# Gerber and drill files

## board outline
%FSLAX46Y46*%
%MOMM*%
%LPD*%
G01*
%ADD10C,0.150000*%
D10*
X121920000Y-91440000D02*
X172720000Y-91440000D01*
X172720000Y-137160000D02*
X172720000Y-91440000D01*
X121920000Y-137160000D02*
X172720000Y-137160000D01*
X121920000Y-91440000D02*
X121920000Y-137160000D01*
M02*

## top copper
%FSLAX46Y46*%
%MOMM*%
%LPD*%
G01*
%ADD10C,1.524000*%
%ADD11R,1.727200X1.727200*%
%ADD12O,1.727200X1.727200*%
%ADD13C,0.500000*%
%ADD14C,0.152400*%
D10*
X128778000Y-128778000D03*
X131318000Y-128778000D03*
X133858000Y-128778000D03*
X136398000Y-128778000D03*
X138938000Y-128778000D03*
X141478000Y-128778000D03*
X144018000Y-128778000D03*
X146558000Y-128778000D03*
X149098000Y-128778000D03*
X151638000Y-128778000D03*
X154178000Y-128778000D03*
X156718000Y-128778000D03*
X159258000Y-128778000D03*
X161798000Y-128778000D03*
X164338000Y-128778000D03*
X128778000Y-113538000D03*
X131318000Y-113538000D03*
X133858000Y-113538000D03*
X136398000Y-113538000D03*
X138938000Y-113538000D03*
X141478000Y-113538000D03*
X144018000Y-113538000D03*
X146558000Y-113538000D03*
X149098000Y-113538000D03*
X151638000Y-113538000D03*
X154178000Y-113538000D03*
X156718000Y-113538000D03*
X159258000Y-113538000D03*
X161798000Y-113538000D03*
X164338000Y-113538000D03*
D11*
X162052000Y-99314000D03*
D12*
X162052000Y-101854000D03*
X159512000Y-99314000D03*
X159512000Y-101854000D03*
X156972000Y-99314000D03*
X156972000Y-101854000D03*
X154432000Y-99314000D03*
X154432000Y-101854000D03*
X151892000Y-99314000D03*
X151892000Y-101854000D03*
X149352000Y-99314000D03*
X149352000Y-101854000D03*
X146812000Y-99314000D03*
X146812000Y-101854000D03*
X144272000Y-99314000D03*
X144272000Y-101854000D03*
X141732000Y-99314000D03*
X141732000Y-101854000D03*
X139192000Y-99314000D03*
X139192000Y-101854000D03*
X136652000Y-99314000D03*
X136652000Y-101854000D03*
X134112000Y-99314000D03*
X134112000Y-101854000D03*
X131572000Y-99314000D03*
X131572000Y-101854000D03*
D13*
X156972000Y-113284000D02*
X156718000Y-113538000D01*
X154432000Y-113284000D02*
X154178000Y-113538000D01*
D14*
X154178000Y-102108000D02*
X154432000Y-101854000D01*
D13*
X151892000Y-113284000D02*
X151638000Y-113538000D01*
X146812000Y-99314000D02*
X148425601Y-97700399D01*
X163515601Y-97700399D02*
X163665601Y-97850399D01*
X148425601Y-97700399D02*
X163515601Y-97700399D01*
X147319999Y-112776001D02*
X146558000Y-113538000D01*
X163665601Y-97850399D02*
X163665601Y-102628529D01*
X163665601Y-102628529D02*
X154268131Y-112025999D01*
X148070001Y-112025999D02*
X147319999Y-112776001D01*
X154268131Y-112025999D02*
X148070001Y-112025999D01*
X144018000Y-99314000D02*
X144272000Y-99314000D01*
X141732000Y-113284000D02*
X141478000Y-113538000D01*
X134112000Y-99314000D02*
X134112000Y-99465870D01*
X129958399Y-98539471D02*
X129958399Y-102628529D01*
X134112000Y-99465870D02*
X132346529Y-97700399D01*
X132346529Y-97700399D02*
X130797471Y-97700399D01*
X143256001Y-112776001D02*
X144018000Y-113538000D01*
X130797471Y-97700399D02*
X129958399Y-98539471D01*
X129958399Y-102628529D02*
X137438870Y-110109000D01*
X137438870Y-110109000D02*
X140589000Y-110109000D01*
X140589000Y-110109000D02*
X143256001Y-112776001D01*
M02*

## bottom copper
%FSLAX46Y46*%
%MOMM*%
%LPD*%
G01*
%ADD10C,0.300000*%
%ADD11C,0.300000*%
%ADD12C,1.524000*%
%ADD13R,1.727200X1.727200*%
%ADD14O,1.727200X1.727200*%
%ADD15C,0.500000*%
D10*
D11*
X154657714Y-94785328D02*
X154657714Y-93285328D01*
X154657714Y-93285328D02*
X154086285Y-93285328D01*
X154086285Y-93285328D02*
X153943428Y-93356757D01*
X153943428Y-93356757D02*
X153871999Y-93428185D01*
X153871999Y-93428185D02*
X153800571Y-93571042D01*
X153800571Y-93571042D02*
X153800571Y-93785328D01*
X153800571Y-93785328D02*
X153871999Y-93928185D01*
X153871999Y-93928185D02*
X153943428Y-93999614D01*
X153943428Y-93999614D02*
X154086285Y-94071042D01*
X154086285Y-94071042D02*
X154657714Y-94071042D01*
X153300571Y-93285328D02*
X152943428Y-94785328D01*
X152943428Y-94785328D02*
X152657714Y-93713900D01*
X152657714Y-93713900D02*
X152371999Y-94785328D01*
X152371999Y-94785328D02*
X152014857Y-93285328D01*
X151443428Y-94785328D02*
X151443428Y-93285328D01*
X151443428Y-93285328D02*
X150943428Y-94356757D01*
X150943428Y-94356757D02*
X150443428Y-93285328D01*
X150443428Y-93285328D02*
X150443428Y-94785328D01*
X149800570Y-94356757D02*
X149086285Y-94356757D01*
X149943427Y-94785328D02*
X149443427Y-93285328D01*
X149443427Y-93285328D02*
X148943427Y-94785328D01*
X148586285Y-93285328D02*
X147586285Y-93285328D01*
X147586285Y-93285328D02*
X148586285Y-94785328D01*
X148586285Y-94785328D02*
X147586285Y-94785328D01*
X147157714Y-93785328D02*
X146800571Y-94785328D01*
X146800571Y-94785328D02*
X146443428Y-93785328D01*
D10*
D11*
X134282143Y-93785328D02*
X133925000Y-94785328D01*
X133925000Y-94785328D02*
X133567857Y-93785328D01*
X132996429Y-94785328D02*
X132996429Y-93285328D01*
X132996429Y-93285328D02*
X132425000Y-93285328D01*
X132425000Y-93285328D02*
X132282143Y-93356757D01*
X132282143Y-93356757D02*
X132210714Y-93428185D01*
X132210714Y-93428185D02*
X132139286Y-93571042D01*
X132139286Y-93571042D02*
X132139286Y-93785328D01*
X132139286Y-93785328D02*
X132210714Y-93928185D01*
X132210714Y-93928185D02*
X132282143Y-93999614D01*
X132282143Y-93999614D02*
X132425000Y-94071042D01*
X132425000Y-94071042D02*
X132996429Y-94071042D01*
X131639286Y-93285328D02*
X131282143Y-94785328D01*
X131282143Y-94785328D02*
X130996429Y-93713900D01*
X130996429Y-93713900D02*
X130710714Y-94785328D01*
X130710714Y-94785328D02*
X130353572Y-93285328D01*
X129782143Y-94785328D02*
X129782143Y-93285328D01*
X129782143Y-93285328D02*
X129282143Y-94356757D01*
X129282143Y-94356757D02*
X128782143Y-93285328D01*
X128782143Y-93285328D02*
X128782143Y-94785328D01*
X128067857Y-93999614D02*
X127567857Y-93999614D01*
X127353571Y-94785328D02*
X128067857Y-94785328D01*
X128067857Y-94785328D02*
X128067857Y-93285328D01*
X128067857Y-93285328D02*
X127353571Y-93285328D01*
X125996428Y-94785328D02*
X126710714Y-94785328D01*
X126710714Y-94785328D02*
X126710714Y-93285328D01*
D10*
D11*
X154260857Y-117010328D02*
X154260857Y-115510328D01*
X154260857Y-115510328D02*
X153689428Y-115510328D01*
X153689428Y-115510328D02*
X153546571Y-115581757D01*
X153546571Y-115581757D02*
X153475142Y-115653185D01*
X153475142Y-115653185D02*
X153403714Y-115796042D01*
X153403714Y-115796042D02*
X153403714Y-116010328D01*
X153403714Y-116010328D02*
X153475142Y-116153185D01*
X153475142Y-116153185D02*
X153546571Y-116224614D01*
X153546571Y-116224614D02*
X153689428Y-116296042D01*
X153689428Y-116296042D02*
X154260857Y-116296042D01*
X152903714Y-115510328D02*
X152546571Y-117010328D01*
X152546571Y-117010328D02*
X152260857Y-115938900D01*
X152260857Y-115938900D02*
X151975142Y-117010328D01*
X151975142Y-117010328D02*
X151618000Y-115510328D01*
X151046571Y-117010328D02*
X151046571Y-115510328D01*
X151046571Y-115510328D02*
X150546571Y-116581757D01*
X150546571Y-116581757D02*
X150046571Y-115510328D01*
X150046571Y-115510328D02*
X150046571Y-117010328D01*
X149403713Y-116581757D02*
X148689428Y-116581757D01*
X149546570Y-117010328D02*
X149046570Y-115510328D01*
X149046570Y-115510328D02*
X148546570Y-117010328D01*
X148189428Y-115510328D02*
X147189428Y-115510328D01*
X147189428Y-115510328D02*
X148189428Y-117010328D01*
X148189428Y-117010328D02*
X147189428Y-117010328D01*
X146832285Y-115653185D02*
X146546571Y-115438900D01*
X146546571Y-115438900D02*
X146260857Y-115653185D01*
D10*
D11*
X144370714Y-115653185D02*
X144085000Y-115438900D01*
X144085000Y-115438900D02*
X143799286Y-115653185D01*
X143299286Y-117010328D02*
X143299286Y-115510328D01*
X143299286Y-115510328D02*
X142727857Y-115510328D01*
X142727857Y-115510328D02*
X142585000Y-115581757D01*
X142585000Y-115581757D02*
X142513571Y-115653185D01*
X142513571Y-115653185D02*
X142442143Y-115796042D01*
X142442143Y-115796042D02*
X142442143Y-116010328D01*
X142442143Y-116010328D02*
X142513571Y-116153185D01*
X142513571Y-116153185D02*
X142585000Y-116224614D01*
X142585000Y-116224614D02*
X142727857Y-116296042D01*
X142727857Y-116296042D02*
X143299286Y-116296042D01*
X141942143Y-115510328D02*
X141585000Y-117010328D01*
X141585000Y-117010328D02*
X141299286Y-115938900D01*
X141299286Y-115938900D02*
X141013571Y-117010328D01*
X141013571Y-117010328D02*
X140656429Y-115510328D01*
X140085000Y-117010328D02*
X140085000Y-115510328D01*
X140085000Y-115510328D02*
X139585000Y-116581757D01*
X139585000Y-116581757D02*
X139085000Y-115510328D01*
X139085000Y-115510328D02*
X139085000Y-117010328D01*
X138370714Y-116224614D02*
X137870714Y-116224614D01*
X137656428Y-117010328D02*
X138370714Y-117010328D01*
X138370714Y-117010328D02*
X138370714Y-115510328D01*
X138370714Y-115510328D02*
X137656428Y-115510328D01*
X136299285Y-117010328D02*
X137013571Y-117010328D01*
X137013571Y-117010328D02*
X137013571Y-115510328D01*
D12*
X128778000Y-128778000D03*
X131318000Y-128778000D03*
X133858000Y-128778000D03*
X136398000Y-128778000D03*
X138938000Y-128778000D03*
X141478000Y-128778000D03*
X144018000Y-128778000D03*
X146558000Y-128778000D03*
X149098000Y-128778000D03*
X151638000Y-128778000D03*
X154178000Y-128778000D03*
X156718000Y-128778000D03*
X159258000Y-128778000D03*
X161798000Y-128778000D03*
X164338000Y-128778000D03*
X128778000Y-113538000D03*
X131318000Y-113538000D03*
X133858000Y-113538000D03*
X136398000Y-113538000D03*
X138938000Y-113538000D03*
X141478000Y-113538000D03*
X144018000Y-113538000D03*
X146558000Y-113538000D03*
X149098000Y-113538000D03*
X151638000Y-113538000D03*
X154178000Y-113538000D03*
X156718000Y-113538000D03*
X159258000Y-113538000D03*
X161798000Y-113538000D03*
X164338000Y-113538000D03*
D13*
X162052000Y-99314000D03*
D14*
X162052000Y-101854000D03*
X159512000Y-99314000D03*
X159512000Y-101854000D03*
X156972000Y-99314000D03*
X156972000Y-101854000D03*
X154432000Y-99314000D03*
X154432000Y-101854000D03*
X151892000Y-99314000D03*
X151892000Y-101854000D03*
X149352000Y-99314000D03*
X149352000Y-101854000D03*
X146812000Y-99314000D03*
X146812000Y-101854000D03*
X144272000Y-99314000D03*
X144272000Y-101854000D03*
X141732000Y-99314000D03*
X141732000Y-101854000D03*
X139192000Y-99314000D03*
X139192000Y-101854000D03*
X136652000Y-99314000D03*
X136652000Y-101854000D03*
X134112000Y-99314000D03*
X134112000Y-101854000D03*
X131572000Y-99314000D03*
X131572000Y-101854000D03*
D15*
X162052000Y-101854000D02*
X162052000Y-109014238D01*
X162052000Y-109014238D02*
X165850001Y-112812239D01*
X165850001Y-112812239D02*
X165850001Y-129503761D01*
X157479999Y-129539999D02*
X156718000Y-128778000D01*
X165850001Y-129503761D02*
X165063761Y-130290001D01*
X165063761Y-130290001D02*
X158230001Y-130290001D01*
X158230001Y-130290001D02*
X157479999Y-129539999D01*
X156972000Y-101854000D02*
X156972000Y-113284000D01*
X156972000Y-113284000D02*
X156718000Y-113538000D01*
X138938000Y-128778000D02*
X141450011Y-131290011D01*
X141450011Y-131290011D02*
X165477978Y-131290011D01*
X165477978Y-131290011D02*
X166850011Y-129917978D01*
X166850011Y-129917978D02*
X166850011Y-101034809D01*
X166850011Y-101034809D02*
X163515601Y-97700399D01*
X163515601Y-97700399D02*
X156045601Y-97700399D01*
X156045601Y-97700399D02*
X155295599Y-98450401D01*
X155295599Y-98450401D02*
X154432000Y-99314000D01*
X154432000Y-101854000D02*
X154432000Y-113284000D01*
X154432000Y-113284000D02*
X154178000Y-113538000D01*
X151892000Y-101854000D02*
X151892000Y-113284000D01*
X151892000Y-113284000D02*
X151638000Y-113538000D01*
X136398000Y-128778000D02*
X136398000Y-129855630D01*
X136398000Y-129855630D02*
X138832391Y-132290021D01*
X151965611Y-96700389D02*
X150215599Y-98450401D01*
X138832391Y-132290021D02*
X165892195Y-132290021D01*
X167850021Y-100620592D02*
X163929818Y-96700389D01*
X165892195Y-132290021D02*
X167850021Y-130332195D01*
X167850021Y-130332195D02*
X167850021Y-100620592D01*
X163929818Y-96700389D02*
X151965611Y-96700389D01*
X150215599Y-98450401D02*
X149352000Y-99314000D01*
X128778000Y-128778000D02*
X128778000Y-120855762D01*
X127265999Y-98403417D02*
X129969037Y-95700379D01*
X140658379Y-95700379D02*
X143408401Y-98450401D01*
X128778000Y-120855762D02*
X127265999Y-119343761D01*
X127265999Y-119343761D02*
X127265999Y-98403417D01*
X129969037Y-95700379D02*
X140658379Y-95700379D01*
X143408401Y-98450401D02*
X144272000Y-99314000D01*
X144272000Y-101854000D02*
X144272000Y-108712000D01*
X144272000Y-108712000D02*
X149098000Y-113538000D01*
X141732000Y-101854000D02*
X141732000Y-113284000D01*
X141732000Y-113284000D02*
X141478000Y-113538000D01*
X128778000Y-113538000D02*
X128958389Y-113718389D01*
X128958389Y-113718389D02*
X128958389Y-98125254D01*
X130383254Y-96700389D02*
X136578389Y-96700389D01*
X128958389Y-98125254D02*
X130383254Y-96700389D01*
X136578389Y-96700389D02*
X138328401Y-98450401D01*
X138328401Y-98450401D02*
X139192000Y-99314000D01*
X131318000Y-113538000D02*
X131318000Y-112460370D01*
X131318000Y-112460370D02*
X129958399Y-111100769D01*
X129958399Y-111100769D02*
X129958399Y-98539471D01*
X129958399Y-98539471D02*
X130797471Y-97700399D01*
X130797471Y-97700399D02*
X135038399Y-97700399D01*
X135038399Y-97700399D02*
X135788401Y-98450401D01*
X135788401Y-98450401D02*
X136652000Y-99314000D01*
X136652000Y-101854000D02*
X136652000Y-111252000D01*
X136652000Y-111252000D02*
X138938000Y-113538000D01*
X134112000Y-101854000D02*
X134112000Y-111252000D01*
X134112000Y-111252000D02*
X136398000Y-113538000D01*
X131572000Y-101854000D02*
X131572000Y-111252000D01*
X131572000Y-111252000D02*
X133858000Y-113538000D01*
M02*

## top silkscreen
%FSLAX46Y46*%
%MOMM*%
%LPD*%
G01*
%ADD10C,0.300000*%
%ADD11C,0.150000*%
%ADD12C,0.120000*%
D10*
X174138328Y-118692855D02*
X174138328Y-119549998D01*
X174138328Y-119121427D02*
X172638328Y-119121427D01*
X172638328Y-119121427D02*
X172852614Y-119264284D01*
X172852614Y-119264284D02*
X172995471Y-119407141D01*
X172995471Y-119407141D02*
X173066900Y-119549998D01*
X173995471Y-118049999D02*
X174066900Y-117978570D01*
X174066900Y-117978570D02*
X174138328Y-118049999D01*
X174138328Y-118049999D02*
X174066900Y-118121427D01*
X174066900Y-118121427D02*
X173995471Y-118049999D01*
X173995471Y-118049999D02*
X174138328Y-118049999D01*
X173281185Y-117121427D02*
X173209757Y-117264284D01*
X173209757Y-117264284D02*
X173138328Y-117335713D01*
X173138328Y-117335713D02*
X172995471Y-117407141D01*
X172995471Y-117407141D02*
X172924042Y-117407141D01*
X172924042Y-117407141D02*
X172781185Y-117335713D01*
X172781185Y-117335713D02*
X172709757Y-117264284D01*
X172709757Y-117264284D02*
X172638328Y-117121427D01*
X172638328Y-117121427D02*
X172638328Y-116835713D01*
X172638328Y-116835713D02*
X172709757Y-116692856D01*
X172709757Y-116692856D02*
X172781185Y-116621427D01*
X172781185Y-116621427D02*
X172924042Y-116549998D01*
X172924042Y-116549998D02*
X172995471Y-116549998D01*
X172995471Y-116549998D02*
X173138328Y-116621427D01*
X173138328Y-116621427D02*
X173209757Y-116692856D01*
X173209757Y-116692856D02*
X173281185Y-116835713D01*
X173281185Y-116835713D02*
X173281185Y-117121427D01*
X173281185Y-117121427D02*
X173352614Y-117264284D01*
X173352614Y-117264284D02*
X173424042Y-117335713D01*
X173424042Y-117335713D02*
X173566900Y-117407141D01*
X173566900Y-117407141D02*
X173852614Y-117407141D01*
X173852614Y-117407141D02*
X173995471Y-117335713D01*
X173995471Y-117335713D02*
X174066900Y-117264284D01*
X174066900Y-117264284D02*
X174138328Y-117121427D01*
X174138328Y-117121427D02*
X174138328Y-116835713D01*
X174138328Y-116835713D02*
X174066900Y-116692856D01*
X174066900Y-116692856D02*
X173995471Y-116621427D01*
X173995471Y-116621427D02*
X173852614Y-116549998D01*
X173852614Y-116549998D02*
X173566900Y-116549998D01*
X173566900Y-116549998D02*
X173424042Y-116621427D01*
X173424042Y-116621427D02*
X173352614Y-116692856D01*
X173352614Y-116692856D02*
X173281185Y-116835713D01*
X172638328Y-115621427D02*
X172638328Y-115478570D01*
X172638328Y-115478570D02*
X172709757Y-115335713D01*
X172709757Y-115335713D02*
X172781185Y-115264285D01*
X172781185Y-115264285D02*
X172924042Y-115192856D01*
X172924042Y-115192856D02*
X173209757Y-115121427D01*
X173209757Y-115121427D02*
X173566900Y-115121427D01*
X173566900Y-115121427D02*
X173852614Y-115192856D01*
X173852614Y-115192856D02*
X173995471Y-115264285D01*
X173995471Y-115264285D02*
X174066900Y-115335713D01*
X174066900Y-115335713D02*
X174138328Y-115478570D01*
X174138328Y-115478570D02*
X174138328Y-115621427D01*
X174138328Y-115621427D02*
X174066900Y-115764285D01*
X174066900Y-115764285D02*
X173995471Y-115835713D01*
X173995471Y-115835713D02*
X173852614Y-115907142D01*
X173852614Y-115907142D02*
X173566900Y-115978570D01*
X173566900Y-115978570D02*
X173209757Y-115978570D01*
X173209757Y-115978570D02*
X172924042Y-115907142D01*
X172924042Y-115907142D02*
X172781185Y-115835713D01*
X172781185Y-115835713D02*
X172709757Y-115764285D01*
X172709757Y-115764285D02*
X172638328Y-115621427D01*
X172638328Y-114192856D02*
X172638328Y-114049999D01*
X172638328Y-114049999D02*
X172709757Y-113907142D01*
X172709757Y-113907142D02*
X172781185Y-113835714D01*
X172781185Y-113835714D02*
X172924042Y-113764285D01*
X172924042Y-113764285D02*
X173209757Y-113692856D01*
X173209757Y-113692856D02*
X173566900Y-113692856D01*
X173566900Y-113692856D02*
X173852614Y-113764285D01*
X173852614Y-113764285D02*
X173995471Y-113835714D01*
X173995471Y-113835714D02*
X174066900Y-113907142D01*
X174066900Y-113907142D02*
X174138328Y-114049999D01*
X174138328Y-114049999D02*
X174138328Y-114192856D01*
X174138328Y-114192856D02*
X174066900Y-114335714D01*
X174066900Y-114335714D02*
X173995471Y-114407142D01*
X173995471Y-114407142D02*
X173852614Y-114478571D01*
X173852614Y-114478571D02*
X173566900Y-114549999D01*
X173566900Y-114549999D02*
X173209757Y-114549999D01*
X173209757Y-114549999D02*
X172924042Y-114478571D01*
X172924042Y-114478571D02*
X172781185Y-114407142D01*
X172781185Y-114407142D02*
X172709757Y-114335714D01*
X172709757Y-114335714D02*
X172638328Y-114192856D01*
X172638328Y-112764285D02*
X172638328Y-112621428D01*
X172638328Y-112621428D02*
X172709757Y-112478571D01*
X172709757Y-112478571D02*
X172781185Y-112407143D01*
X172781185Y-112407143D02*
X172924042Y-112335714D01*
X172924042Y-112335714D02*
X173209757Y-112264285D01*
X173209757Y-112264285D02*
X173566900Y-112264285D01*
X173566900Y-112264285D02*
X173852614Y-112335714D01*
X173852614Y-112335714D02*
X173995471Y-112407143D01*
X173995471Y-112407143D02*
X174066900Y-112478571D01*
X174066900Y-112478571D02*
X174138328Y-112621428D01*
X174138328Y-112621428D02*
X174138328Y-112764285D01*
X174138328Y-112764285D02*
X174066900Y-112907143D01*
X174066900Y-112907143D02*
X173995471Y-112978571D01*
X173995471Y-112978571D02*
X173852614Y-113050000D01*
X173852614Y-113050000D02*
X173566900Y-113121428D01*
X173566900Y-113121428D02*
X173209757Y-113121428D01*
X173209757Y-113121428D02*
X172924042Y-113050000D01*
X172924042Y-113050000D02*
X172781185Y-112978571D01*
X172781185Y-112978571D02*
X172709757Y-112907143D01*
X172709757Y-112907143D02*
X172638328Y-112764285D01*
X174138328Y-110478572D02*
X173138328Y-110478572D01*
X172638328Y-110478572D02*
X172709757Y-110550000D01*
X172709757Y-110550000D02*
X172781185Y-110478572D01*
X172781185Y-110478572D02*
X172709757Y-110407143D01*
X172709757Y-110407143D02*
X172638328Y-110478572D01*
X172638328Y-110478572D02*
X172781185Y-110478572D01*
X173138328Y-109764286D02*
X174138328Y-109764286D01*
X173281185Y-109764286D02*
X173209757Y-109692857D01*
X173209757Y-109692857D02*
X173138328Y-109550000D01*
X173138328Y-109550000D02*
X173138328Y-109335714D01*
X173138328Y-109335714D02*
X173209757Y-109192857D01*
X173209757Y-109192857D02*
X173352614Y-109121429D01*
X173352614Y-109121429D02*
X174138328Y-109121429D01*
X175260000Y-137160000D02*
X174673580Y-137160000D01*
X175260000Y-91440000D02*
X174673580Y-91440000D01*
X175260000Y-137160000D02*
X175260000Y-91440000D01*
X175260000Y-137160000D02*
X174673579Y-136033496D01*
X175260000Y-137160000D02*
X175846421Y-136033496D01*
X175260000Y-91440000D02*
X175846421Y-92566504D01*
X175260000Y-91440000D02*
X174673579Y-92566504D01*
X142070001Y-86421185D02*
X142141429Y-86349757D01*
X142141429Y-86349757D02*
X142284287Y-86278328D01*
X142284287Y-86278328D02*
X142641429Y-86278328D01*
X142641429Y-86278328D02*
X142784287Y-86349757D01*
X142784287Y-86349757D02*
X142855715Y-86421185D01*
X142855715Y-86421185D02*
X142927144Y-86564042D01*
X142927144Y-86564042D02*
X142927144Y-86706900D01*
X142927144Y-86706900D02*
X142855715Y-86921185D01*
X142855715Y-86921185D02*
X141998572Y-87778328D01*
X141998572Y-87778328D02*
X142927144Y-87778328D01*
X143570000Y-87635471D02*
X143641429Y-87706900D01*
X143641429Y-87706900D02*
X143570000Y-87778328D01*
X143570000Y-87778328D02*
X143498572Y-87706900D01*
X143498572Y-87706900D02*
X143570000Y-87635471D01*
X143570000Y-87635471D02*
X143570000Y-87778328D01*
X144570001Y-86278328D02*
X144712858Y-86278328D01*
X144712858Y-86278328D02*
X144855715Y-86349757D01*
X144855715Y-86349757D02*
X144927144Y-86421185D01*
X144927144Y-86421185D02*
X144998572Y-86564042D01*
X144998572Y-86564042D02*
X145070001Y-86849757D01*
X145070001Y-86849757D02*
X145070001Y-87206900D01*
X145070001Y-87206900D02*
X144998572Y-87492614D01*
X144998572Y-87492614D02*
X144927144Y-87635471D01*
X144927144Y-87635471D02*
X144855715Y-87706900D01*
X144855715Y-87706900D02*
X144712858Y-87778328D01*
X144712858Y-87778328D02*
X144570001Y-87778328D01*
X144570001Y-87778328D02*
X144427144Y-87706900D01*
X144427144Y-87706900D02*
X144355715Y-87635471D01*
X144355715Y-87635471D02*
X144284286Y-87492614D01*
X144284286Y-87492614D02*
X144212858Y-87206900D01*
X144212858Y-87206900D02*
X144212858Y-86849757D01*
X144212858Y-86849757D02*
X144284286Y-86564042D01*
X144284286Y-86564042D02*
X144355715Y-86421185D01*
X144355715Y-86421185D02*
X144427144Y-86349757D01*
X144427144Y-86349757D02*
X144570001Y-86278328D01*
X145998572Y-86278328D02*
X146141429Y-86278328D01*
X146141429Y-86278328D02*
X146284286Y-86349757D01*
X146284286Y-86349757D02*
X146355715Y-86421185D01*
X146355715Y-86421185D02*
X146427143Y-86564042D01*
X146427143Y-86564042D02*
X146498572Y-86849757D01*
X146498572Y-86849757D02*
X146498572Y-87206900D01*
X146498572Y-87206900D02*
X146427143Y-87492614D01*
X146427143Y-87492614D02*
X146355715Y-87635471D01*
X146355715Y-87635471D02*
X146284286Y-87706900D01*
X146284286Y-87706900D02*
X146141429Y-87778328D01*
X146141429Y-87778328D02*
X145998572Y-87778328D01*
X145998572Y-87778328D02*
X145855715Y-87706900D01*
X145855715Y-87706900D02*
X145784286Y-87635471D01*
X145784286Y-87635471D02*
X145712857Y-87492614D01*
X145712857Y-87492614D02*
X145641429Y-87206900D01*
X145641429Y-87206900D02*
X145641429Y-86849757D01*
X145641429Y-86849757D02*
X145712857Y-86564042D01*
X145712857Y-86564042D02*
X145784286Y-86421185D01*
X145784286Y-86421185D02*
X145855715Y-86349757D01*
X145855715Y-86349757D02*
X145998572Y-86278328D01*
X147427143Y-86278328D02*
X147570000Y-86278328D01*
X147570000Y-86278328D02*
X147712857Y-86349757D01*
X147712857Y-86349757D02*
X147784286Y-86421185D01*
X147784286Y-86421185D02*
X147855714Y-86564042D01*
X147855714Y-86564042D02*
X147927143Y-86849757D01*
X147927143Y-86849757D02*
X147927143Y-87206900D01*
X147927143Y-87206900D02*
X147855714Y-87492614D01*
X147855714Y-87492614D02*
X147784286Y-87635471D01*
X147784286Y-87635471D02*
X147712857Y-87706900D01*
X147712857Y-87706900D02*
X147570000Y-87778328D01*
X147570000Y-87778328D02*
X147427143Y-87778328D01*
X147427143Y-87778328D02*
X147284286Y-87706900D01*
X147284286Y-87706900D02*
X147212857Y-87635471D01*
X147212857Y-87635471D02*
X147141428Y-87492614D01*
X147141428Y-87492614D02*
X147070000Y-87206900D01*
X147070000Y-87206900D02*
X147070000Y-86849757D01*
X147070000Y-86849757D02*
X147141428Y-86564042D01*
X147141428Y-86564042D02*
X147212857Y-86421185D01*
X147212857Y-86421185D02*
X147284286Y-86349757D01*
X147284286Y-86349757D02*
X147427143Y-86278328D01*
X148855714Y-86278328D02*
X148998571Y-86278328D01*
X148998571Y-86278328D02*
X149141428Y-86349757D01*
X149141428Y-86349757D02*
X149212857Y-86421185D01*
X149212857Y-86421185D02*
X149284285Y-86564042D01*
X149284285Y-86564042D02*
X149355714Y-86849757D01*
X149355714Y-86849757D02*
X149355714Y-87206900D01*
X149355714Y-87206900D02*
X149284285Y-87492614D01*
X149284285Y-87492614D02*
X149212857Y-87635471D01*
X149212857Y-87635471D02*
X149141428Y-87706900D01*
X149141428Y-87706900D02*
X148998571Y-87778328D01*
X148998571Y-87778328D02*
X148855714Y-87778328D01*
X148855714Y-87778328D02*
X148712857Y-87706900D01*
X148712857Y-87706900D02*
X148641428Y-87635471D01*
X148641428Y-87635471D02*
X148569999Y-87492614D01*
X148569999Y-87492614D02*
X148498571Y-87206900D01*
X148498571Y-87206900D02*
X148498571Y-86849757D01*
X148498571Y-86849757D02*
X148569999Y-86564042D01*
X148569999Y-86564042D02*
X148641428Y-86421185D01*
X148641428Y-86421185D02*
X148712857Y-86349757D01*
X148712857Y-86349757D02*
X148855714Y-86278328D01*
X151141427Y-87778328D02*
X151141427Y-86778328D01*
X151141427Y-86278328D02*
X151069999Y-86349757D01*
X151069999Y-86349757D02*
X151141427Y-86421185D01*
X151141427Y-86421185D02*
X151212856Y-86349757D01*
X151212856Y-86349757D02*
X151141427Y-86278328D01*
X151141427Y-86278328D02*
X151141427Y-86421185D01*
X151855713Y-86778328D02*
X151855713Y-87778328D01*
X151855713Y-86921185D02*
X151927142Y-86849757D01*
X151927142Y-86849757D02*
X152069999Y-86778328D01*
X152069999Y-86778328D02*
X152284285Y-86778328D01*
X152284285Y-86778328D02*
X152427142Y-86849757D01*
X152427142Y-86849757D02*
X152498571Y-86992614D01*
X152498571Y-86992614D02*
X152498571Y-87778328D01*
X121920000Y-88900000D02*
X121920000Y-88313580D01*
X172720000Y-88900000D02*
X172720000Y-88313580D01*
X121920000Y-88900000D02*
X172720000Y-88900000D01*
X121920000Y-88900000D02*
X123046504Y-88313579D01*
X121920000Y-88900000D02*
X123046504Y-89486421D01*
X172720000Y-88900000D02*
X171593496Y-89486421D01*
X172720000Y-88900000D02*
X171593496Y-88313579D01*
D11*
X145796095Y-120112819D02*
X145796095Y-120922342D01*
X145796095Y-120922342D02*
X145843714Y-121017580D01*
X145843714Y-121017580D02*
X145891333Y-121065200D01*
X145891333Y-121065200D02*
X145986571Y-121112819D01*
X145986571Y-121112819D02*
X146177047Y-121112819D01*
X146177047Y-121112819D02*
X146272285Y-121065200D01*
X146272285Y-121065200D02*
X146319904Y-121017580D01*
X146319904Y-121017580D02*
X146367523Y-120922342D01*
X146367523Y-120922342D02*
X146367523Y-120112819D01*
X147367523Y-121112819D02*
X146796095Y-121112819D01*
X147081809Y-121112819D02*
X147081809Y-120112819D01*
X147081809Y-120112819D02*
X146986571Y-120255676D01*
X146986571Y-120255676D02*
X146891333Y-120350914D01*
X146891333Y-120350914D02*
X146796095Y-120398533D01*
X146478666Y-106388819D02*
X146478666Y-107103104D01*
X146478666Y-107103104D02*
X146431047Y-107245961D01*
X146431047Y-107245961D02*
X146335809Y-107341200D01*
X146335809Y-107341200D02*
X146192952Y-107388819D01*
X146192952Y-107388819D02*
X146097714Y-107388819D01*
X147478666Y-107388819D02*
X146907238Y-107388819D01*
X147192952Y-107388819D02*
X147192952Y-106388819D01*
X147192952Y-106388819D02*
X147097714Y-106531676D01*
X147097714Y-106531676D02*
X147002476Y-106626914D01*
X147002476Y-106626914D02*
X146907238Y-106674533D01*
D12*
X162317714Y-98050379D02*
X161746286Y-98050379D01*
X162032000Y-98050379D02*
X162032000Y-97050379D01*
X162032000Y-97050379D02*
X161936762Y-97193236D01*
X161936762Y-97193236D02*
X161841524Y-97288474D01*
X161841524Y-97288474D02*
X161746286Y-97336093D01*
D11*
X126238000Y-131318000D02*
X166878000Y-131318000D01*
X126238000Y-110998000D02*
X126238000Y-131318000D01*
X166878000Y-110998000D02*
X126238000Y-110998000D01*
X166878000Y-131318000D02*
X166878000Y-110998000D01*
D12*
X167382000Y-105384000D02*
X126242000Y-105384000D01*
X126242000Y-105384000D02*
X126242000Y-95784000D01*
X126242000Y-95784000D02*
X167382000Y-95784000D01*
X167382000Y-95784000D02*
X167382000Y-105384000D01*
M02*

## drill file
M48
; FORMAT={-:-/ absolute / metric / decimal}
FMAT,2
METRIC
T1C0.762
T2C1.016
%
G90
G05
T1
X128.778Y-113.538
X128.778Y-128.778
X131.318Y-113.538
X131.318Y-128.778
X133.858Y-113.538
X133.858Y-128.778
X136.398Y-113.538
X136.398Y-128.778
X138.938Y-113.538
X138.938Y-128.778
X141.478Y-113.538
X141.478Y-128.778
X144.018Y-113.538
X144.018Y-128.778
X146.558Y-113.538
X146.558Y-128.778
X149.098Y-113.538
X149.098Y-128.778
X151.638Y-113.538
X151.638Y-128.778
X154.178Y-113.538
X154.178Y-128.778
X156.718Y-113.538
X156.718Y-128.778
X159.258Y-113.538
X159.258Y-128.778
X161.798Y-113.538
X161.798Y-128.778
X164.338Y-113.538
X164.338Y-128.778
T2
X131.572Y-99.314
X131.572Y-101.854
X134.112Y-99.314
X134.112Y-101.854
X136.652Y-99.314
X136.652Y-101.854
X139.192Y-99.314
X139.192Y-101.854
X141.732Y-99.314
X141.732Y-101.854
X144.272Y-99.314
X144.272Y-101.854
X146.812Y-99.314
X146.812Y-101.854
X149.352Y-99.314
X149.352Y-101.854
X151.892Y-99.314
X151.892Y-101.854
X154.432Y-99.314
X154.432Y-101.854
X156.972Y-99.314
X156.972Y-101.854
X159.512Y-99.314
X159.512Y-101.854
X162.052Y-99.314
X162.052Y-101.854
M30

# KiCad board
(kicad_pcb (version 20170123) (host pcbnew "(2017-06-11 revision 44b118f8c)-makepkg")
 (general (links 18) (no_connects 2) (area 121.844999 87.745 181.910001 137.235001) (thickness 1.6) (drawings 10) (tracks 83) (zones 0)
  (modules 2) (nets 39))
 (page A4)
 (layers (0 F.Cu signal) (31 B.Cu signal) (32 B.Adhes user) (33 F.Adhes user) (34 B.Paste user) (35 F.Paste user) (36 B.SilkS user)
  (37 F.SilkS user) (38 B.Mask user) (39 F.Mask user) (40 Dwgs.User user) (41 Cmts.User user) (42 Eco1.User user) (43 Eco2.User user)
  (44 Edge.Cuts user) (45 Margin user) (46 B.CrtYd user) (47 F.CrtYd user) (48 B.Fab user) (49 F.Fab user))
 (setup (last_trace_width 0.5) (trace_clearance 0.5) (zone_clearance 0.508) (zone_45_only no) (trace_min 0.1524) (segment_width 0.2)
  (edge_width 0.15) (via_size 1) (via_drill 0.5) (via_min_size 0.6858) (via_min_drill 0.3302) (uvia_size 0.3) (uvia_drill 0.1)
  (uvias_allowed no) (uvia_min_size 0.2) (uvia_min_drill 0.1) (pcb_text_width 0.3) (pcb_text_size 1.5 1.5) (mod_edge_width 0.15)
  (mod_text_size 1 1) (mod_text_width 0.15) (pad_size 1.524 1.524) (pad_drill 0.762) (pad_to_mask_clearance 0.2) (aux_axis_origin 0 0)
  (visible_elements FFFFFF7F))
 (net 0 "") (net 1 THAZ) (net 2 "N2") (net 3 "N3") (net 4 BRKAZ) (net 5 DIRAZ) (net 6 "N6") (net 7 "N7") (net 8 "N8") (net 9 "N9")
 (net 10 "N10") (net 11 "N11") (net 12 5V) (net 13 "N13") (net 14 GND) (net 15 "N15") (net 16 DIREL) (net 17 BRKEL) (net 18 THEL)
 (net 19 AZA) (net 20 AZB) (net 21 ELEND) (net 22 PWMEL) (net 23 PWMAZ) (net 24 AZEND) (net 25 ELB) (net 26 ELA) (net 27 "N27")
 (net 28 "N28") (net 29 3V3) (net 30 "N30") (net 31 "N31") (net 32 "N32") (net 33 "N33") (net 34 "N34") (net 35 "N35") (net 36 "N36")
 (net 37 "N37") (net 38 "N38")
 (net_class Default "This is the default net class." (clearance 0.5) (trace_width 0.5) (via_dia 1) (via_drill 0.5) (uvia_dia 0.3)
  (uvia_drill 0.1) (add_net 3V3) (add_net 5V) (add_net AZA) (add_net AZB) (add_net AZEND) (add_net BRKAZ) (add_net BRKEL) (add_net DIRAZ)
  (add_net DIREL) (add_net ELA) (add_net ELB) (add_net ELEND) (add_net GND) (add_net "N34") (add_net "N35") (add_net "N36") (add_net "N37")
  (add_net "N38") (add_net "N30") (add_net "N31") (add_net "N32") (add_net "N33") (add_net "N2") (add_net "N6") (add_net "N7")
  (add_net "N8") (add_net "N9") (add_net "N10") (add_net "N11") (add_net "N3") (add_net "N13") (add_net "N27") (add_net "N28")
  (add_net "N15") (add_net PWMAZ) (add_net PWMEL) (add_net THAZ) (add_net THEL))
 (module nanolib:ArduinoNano (layer F.Cu) (at 146.558 121.158 180)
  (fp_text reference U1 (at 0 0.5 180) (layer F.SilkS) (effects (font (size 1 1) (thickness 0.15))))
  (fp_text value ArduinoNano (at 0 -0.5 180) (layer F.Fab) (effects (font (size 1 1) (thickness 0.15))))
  (fp_line (start 20.32 -10.16) (end -20.32 -10.16) (layer F.SilkS) (width 0.15))
  (fp_line (start 20.32 10.16) (end 20.32 -10.16) (layer F.SilkS) (width 0.15))
  (fp_line (start -20.32 10.16) (end 20.32 10.16) (layer F.SilkS) (width 0.15))
  (fp_line (start -20.32 -10.16) (end -20.32 10.16) (layer F.SilkS) (width 0.15))
  (pad D13 thru_hole circle (at 17.78 -7.62 180) (size 1.524 1.524) (drill 0.762) (layers *.Cu *.Mask) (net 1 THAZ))
  (pad 3V3 thru_hole circle (at 15.24 -7.62 180) (size 1.524 1.524) (drill 0.762) (layers *.Cu *.Mask) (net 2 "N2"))
  (pad REF thru_hole circle (at 12.7 -7.62 180) (size 1.524 1.524) (drill 0.762) (layers *.Cu *.Mask) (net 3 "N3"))
  (pad A0 thru_hole circle (at 10.16 -7.62 180) (size 1.524 1.524) (drill 0.762) (layers *.Cu *.Mask) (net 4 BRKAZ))
  (pad A1 thru_hole circle (at 7.62 -7.62 180) (size 1.524 1.524) (drill 0.762) (layers *.Cu *.Mask) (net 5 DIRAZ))
  (pad A2 thru_hole circle (at 5.08 -7.62 180) (size 1.524 1.524) (drill 0.762) (layers *.Cu *.Mask) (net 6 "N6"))
  (pad A3 thru_hole circle (at 2.54 -7.62 180) (size 1.524 1.524) (drill 0.762) (layers *.Cu *.Mask) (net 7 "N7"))
  (pad A4 thru_hole circle (at 0 -7.62 180) (size 1.524 1.524) (drill 0.762) (layers *.Cu *.Mask) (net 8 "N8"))
  (pad A5 thru_hole circle (at -2.54 -7.62 180) (size 1.524 1.524) (drill 0.762) (layers *.Cu *.Mask) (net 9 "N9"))
  (pad A6 thru_hole circle (at -5.08 -7.62 180) (size 1.524 1.524) (drill 0.762) (layers *.Cu *.Mask) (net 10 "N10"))
  (pad A7 thru_hole circle (at -7.62 -7.62 180) (size 1.524 1.524) (drill 0.762) (layers *.Cu *.Mask) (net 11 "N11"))
  (pad 5V thru_hole circle (at -10.16 -7.62 180) (size 1.524 1.524) (drill 0.762) (layers *.Cu *.Mask) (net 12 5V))
  (pad RST thru_hole circle (at -12.7 -7.62 180) (size 1.524 1.524) (drill 0.762) (layers *.Cu *.Mask) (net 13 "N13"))
  (pad GND thru_hole circle (at -15.24 -7.62 180) (size 1.524 1.524) (drill 0.762) (layers *.Cu *.Mask) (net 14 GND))
  (pad VIN thru_hole circle (at -17.78 -7.62 180) (size 1.524 1.524) (drill 0.762) (layers *.Cu *.Mask) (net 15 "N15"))
  (pad D12 thru_hole circle (at 17.78 7.62 180) (size 1.524 1.524) (drill 0.762) (layers *.Cu *.Mask) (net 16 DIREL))
  (pad D11 thru_hole circle (at 15.24 7.62 180) (size 1.524 1.524) (drill 0.762) (layers *.Cu *.Mask) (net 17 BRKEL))
  (pad D10 thru_hole circle (at 12.7 7.62 180) (size 1.524 1.524) (drill 0.762) (layers *.Cu *.Mask) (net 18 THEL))
  (pad D9 thru_hole circle (at 10.16 7.62 180) (size 1.524 1.524) (drill 0.762) (layers *.Cu *.Mask) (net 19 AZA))
  (pad D8 thru_hole circle (at 7.62 7.62 180) (size 1.524 1.524) (drill 0.762) (layers *.Cu *.Mask) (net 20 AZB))
  (pad D7 thru_hole circle (at 5.08 7.62 180) (size 1.524 1.524) (drill 0.762) (layers *.Cu *.Mask) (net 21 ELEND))
  (pad D6 thru_hole circle (at 2.54 7.62 180) (size 1.524 1.524) (drill 0.762) (layers *.Cu *.Mask) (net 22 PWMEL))
  (pad D5 thru_hole circle (at 0 7.62 180) (size 1.524 1.524) (drill 0.762) (layers *.Cu *.Mask) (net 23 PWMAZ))
  (pad D4 thru_hole circle (at -2.54 7.62 180) (size 1.524 1.524) (drill 0.762) (layers *.Cu *.Mask) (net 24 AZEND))
  (pad D3 thru_hole circle (at -5.08 7.62 180) (size 1.524 1.524) (drill 0.762) (layers *.Cu *.Mask) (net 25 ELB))
  (pad D2 thru_hole circle (at -7.62 7.62 180) (size 1.524 1.524) (drill 0.762) (layers *.Cu *.Mask) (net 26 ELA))
  (pad GND thru_hole circle (at -10.16 7.62 180) (size 1.524 1.524) (drill 0.762) (layers *.Cu *.Mask) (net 14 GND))
  (pad RST thru_hole circle (at -12.7 7.62 180) (size 1.524 1.524) (drill 0.762) (layers *.Cu *.Mask) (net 13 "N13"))
  (pad RX0 thru_hole circle (at -15.24 7.62 180) (size 1.524 1.524) (drill 0.762) (layers *.Cu *.Mask) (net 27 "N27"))
  (pad TX1 thru_hole circle (at -17.78 7.62 180) (size 1.524 1.524) (drill 0.762) (layers *.Cu *.Mask) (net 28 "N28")))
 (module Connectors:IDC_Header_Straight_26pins (layer F.Cu) (at 162.052 99.314 180)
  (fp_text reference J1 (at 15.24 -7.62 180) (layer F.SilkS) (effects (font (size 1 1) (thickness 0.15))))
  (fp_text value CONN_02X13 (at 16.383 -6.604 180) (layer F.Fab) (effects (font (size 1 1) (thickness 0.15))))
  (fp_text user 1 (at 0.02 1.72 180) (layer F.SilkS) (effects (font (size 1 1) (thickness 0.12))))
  (fp_line (start -5.33 -6.07) (end 35.81 -6.07) (layer F.SilkS) (width 0.12))
  (fp_line (start 35.81 -6.07) (end 35.81 3.53) (layer F.SilkS) (width 0.12))
  (fp_line (start 35.81 3.53) (end -5.33 3.53) (layer F.SilkS) (width 0.12))
  (fp_line (start -5.33 3.53) (end -5.33 -6.07) (layer F.SilkS) (width 0.12))
  (pad 1 thru_hole rect (at 0 0 180) (size 1.7272 1.7272) (drill 1.016) (layers *.Cu *.Mask) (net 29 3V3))
  (pad 2 thru_hole oval (at 0 -2.54 180) (size 1.7272 1.7272) (drill 1.016) (layers *.Cu *.Mask) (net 12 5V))
  (pad 3 thru_hole oval (at 2.54 0 180) (size 1.7272 1.7272) (drill 1.016) (layers *.Cu *.Mask) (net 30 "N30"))
  (pad 4 thru_hole oval (at 2.54 -2.54 180) (size 1.7272 1.7272) (drill 1.016) (layers *.Cu *.Mask) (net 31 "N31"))
  (pad 5 thru_hole oval (at 5.08 0 180) (size 1.7272 1.7272) (drill 1.016) (layers *.Cu *.Mask) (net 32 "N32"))
  (pad 6 thru_hole oval (at 5.08 -2.54 180) (size 1.7272 1.7272) (drill 1.016) (layers *.Cu *.Mask) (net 14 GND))
  (pad 7 thru_hole oval (at 7.62 0 180) (size 1.7272 1.7272) (drill 1.016) (layers *.Cu *.Mask) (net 5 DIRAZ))
  (pad 8 thru_hole oval (at 7.62 -2.54 180) (size 1.7272 1.7272) (drill 1.016) (layers *.Cu *.Mask) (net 26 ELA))
  (pad 9 thru_hole oval (at 10.16 0 180) (size 1.7272 1.7272) (drill 1.016) (layers *.Cu *.Mask) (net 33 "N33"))
  (pad 10 thru_hole oval (at 10.16 -2.54 180) (size 1.7272 1.7272) (drill 1.016) (layers *.Cu *.Mask) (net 25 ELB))
  (pad 11 thru_hole oval (at 12.7 0 180) (size 1.7272 1.7272) (drill 1.016) (layers *.Cu *.Mask) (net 4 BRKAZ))
  (pad 12 thru_hole oval (at 12.7 -2.54 180) (size 1.7272 1.7272) (drill 1.016) (layers *.Cu *.Mask) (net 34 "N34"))
  (pad 13 thru_hole oval (at 15.24 0 180) (size 1.7272 1.7272) (drill 1.016) (layers *.Cu *.Mask) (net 23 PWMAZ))
  (pad 14 thru_hole oval (at 15.24 -2.54 180) (size 1.7272 1.7272) (drill 1.016) (layers *.Cu *.Mask) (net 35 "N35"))
  (pad 15 thru_hole oval (at 17.78 0 180) (size 1.7272 1.7272) (drill 1.016) (layers *.Cu *.Mask) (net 1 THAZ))
  (pad 16 thru_hole oval (at 17.78 -2.54 180) (size 1.7272 1.7272) (drill 1.016) (layers *.Cu *.Mask) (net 24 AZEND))
  (pad 17 thru_hole oval (at 20.32 0 180) (size 1.7272 1.7272) (drill 1.016) (layers *.Cu *.Mask) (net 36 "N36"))
  (pad 18 thru_hole oval (at 20.32 -2.54 180) (size 1.7272 1.7272) (drill 1.016) (layers *.Cu *.Mask) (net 21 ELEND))
  (pad 19 thru_hole oval (at 22.86 0 180) (size 1.7272 1.7272) (drill 1.016) (layers *.Cu *.Mask) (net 16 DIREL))
  (pad 20 thru_hole oval (at 22.86 -2.54 180) (size 1.7272 1.7272) (drill 1.016) (layers *.Cu *.Mask) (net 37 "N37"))
  (pad 21 thru_hole oval (at 25.4 0 180) (size 1.7272 1.7272) (drill 1.016) (layers *.Cu *.Mask) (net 17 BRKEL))
  (pad 22 thru_hole oval (at 25.4 -2.54 180) (size 1.7272 1.7272) (drill 1.016) (layers *.Cu *.Mask) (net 20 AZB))
  (pad 23 thru_hole oval (at 27.94 0 180) (size 1.7272 1.7272) (drill 1.016) (layers *.Cu *.Mask) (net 22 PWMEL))
  (pad 24 thru_hole oval (at 27.94 -2.54 180) (size 1.7272 1.7272) (drill 1.016) (layers *.Cu *.Mask) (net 19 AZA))
  (pad 25 thru_hole oval (at 30.48 0 180) (size 1.7272 1.7272) (drill 1.016) (layers *.Cu *.Mask) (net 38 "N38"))
  (pad 26 thru_hole oval (at 30.48 -2.54 180) (size 1.7272 1.7272) (drill 1.016) (layers *.Cu *.Mask) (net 18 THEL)))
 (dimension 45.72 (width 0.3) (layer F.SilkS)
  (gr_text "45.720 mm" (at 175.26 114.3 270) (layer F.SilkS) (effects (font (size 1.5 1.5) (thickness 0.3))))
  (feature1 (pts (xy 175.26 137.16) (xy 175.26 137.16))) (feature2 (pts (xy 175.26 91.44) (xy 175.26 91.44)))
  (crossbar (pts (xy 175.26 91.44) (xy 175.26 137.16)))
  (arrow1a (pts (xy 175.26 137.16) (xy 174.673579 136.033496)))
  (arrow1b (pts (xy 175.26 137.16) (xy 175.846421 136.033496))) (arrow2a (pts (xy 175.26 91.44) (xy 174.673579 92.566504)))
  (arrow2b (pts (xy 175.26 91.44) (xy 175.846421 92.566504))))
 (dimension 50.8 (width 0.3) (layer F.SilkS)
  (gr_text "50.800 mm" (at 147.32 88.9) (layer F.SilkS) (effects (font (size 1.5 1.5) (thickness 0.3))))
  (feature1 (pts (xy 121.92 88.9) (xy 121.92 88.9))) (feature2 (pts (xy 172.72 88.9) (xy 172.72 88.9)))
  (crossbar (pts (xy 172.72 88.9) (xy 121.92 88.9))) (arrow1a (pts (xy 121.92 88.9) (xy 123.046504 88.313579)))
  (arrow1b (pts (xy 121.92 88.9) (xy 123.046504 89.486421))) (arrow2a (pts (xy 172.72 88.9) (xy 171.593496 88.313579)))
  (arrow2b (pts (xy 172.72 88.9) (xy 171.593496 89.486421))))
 (gr_line (start 121.92 91.44) (end 172.72 91.44) (layer Edge.Cuts) (width 0.15))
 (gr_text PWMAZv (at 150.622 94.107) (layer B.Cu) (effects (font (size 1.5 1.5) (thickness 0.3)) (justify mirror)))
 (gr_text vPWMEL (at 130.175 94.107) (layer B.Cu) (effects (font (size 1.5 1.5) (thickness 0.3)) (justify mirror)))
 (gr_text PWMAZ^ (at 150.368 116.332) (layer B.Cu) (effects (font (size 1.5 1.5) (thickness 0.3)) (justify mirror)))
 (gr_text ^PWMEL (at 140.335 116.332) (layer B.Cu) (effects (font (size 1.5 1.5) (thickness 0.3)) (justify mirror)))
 (gr_line (start 172.72 137.16) (end 172.72 91.44) (layer Edge.Cuts) (width 0.15))
 (gr_line (start 121.92 137.16) (end 172.72 137.16) (layer Edge.Cuts) (width 0.15))
 (gr_line (start 121.92 91.44) (end 121.92 137.16) (layer Edge.Cuts) (width 0.15))
 (segment (start 162.052 101.854) (end 162.052 109.014238) (width 0.5) (layer B.Cu) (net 12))
 (segment (start 162.052 109.014238) (end 165.850001 112.812239) (width 0.5) (layer B.Cu) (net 12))
 (segment (start 165.850001 112.812239) (end 165.850001 129.503761) (width 0.5) (layer B.Cu) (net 12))
 (segment (start 157.479999 129.539999) (end 156.718 128.778) (width 0.5) (layer B.Cu) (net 12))
 (segment (start 165.850001 129.503761) (end 165.063761 130.290001) (width 0.5) (layer B.Cu) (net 12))
 (segment (start 165.063761 130.290001) (end 158.230001 130.290001) (width 0.5) (layer B.Cu) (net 12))
 (segment (start 158.230001 130.290001) (end 157.479999 129.539999) (width 0.5) (layer B.Cu) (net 12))
 (segment (start 156.972 101.854) (end 156.972 113.284) (width 0.5) (layer B.Cu) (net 14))
 (segment (start 156.972 113.284) (end 156.718 113.538) (width 0.5) (layer B.Cu) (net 14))
 (segment (start 156.972 113.284) (end 156.718 113.538) (width 0.5) (layer F.Cu) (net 14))
 (segment (start 138.938 128.778) (end 141.450011 131.290011) (width 0.5) (layer B.Cu) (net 5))
 (segment (start 141.450011 131.290011) (end 165.477978 131.290011) (width 0.5) (layer B.Cu) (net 5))
 (segment (start 165.477978 131.290011) (end 166.850011 129.917978) (width 0.5) (layer B.Cu) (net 5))
 (segment (start 166.850011 129.917978) (end 166.850011 101.034809) (width 0.5) (layer B.Cu) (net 5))
 (segment (start 166.850011 101.034809) (end 163.515601 97.700399) (width 0.5) (layer B.Cu) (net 5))
 (segment (start 163.515601 97.700399) (end 156.045601 97.700399) (width 0.5) (layer B.Cu) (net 5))
 (segment (start 156.045601 97.700399) (end 155.295599 98.450401) (width 0.5) (layer B.Cu) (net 5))
 (segment (start 155.295599 98.450401) (end 154.432 99.314) (width 0.5) (layer B.Cu) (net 5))
 (segment (start 154.432 101.854) (end 154.432 113.284) (width 0.5) (layer B.Cu) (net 26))
 (segment (start 154.432 113.284) (end 154.178 113.538) (width 0.5) (layer B.Cu) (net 26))
 (segment (start 154.432 113.284) (end 154.178 113.538) (width 0.5) (layer F.Cu) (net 26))
 (segment (start 154.178 102.108) (end 154.432 101.854) (width 0.1524) (layer F.Cu) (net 26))
 (segment (start 151.892 101.854) (end 151.892 113.284) (width 0.5) (layer B.Cu) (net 25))
 (segment (start 151.892 113.284) (end 151.638 113.538) (width 0.5) (layer B.Cu) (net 25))
 (segment (start 151.892 113.284) (end 151.638 113.538) (width 0.5) (layer F.Cu) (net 25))
 (segment (start 136.398 128.778) (end 136.398 129.85563) (width 0.5) (layer B.Cu) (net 4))
 (segment (start 136.398 129.85563) (end 138.832391 132.290021) (width 0.5) (layer B.Cu) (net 4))
 (segment (start 151.965611 96.700389) (end 150.215599 98.450401) (width 0.5) (layer B.Cu) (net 4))
 (segment (start 138.832391 132.290021) (end 165.892195 132.290021) (width 0.5) (layer B.Cu) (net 4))
 (segment (start 167.850021 100.620592) (end 163.929818 96.700389) (width 0.5) (layer B.Cu) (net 4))
 (segment (start 165.892195 132.290021) (end 167.850021 130.332195) (width 0.5) (layer B.Cu) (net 4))
 (segment (start 167.850021 130.332195) (end 167.850021 100.620592) (width 0.5) (layer B.Cu) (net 4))
 (segment (start 163.929818 96.700389) (end 151.965611 96.700389) (width 0.5) (layer B.Cu) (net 4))
 (segment (start 150.215599 98.450401) (end 149.352 99.314) (width 0.5) (layer B.Cu) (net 4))
 (segment (start 146.812 99.314) (end 148.425601 97.700399) (width 0.5) (layer F.Cu) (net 23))
 (segment (start 163.515601 97.700399) (end 163.665601 97.850399) (width 0.5) (layer F.Cu) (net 23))
 (segment (start 148.425601 97.700399) (end 163.515601 97.700399) (width 0.5) (layer F.Cu) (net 23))
 (segment (start 147.319999 112.776001) (end 146.558 113.538) (width 0.5) (layer F.Cu) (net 23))
 (segment (start 163.665601 97.850399) (end 163.665601 102.628529) (width 0.5) (layer F.Cu) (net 23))
 (segment (start 163.665601 102.628529) (end 154.268131 112.025999) (width 0.5) (layer F.Cu) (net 23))
 (segment (start 148.070001 112.025999) (end 147.319999 112.776001) (width 0.5) (layer F.Cu) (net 23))
 (segment (start 154.268131 112.025999) (end 148.070001 112.025999) (width 0.5) (layer F.Cu) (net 23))
 (segment (start 128.778 128.778) (end 128.778 120.855762) (width 0.5) (layer B.Cu) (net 1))
 (segment (start 127.265999 98.403417) (end 129.969037 95.700379) (width 0.5) (layer B.Cu) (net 1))
 (segment (start 140.658379 95.700379) (end 143.408401 98.450401) (width 0.5) (layer B.Cu) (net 1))
 (segment (start 128.778 120.855762) (end 127.265999 119.343761) (width 0.5) (layer B.Cu) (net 1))
 (segment (start 127.265999 119.343761) (end 127.265999 98.403417) (width 0.5) (layer B.Cu) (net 1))
 (segment (start 129.969037 95.700379) (end 140.658379 95.700379) (width 0.5) (layer B.Cu) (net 1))
 (segment (start 143.408401 98.450401) (end 144.272 99.314) (width 0.5) (layer B.Cu) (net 1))
 (segment (start 144.018 99.314) (end 144.272 99.314) (width 0.5) (layer F.Cu) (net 1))
 (segment (start 144.272 101.854) (end 144.272 108.712) (width 0.5) (layer B.Cu) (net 24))
 (segment (start 144.272 108.712) (end 149.098 113.538) (width 0.5) (layer B.Cu) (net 24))
 (segment (start 141.732 101.854) (end 141.732 113.284) (width 0.5) (layer B.Cu) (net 21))
 (segment (start 141.732 113.284) (end 141.478 113.538) (width 0.5) (layer B.Cu) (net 21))
 (segment (start 141.732 113.284) (end 141.478 113.538) (width 0.5) (layer F.Cu) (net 21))
 (segment (start 128.778 113.538) (end 128.958389 113.718389) (width 0.5) (layer B.Cu) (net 16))
 (segment (start 128.958389 113.718389) (end 128.958389 98.125254) (width 0.5) (layer B.Cu) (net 16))
 (segment (start 130.383254 96.700389) (end 136.578389 96.700389) (width 0.5) (layer B.Cu) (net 16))
 (segment (start 128.958389 98.125254) (end 130.383254 96.700389) (width 0.5) (layer B.Cu) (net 16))
 (segment (start 136.578389 96.700389) (end 138.328401 98.450401) (width 0.5) (layer B.Cu) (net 16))
 (segment (start 138.328401 98.450401) (end 139.192 99.314) (width 0.5) (layer B.Cu) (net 16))
 (segment (start 131.318 113.538) (end 131.318 112.46037) (width 0.5) (layer B.Cu) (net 17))
 (segment (start 131.318 112.46037) (end 129.958399 111.100769) (width 0.5) (layer B.Cu) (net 17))
 (segment (start 129.958399 111.100769) (end 129.958399 98.539471) (width 0.5) (layer B.Cu) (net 17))
 (segment (start 129.958399 98.539471) (end 130.797471 97.700399) (width 0.5) (layer B.Cu) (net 17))
 (segment (start 130.797471 97.700399) (end 135.038399 97.700399) (width 0.5) (layer B.Cu) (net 17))
 (segment (start 135.038399 97.700399) (end 135.788401 98.450401) (width 0.5) (layer B.Cu) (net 17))
 (segment (start 135.788401 98.450401) (end 136.652 99.314) (width 0.5) (layer B.Cu) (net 17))
 (segment (start 136.652 101.854) (end 136.652 111.252) (width 0.5) (layer B.Cu) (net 20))
 (segment (start 136.652 111.252) (end 138.938 113.538) (width 0.5) (layer B.Cu) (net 20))
 (segment (start 134.112 99.314) (end 134.112 99.46587) (width 0.5) (layer F.Cu) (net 22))
 (segment (start 129.958399 98.539471) (end 129.958399 102.628529) (width 0.5) (layer F.Cu) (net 22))
 (segment (start 134.112 99.46587) (end 132.346529 97.700399) (width 0.5) (layer F.Cu) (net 22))
 (segment (start 132.346529 97.700399) (end 130.797471 97.700399) (width 0.5) (layer F.Cu) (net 22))
 (segment (start 143.256001 112.776001) (end 144.018 113.538) (width 0.5) (layer F.Cu) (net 22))
 (segment (start 130.797471 97.700399) (end 129.958399 98.539471) (width 0.5) (layer F.Cu) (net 22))
 (segment (start 129.958399 102.628529) (end 137.43887 110.109) (width 0.5) (layer F.Cu) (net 22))
 (segment (start 137.43887 110.109) (end 140.589 110.109) (width 0.5) (layer F.Cu) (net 22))
 (segment (start 140.589 110.109) (end 143.256001 112.776001) (width 0.5) (layer F.Cu) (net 22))
 (segment (start 134.112 101.854) (end 134.112 111.252) (width 0.5) (layer B.Cu) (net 19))
 (segment (start 134.112 111.252) (end 136.398 113.538) (width 0.5) (layer B.Cu) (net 19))
 (segment (start 131.572 101.854) (end 131.572 111.252) (width 0.5) (layer B.Cu) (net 18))
 (segment (start 131.572 111.252) (end 133.858 113.538) (width 0.5) (layer B.Cu) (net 18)))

